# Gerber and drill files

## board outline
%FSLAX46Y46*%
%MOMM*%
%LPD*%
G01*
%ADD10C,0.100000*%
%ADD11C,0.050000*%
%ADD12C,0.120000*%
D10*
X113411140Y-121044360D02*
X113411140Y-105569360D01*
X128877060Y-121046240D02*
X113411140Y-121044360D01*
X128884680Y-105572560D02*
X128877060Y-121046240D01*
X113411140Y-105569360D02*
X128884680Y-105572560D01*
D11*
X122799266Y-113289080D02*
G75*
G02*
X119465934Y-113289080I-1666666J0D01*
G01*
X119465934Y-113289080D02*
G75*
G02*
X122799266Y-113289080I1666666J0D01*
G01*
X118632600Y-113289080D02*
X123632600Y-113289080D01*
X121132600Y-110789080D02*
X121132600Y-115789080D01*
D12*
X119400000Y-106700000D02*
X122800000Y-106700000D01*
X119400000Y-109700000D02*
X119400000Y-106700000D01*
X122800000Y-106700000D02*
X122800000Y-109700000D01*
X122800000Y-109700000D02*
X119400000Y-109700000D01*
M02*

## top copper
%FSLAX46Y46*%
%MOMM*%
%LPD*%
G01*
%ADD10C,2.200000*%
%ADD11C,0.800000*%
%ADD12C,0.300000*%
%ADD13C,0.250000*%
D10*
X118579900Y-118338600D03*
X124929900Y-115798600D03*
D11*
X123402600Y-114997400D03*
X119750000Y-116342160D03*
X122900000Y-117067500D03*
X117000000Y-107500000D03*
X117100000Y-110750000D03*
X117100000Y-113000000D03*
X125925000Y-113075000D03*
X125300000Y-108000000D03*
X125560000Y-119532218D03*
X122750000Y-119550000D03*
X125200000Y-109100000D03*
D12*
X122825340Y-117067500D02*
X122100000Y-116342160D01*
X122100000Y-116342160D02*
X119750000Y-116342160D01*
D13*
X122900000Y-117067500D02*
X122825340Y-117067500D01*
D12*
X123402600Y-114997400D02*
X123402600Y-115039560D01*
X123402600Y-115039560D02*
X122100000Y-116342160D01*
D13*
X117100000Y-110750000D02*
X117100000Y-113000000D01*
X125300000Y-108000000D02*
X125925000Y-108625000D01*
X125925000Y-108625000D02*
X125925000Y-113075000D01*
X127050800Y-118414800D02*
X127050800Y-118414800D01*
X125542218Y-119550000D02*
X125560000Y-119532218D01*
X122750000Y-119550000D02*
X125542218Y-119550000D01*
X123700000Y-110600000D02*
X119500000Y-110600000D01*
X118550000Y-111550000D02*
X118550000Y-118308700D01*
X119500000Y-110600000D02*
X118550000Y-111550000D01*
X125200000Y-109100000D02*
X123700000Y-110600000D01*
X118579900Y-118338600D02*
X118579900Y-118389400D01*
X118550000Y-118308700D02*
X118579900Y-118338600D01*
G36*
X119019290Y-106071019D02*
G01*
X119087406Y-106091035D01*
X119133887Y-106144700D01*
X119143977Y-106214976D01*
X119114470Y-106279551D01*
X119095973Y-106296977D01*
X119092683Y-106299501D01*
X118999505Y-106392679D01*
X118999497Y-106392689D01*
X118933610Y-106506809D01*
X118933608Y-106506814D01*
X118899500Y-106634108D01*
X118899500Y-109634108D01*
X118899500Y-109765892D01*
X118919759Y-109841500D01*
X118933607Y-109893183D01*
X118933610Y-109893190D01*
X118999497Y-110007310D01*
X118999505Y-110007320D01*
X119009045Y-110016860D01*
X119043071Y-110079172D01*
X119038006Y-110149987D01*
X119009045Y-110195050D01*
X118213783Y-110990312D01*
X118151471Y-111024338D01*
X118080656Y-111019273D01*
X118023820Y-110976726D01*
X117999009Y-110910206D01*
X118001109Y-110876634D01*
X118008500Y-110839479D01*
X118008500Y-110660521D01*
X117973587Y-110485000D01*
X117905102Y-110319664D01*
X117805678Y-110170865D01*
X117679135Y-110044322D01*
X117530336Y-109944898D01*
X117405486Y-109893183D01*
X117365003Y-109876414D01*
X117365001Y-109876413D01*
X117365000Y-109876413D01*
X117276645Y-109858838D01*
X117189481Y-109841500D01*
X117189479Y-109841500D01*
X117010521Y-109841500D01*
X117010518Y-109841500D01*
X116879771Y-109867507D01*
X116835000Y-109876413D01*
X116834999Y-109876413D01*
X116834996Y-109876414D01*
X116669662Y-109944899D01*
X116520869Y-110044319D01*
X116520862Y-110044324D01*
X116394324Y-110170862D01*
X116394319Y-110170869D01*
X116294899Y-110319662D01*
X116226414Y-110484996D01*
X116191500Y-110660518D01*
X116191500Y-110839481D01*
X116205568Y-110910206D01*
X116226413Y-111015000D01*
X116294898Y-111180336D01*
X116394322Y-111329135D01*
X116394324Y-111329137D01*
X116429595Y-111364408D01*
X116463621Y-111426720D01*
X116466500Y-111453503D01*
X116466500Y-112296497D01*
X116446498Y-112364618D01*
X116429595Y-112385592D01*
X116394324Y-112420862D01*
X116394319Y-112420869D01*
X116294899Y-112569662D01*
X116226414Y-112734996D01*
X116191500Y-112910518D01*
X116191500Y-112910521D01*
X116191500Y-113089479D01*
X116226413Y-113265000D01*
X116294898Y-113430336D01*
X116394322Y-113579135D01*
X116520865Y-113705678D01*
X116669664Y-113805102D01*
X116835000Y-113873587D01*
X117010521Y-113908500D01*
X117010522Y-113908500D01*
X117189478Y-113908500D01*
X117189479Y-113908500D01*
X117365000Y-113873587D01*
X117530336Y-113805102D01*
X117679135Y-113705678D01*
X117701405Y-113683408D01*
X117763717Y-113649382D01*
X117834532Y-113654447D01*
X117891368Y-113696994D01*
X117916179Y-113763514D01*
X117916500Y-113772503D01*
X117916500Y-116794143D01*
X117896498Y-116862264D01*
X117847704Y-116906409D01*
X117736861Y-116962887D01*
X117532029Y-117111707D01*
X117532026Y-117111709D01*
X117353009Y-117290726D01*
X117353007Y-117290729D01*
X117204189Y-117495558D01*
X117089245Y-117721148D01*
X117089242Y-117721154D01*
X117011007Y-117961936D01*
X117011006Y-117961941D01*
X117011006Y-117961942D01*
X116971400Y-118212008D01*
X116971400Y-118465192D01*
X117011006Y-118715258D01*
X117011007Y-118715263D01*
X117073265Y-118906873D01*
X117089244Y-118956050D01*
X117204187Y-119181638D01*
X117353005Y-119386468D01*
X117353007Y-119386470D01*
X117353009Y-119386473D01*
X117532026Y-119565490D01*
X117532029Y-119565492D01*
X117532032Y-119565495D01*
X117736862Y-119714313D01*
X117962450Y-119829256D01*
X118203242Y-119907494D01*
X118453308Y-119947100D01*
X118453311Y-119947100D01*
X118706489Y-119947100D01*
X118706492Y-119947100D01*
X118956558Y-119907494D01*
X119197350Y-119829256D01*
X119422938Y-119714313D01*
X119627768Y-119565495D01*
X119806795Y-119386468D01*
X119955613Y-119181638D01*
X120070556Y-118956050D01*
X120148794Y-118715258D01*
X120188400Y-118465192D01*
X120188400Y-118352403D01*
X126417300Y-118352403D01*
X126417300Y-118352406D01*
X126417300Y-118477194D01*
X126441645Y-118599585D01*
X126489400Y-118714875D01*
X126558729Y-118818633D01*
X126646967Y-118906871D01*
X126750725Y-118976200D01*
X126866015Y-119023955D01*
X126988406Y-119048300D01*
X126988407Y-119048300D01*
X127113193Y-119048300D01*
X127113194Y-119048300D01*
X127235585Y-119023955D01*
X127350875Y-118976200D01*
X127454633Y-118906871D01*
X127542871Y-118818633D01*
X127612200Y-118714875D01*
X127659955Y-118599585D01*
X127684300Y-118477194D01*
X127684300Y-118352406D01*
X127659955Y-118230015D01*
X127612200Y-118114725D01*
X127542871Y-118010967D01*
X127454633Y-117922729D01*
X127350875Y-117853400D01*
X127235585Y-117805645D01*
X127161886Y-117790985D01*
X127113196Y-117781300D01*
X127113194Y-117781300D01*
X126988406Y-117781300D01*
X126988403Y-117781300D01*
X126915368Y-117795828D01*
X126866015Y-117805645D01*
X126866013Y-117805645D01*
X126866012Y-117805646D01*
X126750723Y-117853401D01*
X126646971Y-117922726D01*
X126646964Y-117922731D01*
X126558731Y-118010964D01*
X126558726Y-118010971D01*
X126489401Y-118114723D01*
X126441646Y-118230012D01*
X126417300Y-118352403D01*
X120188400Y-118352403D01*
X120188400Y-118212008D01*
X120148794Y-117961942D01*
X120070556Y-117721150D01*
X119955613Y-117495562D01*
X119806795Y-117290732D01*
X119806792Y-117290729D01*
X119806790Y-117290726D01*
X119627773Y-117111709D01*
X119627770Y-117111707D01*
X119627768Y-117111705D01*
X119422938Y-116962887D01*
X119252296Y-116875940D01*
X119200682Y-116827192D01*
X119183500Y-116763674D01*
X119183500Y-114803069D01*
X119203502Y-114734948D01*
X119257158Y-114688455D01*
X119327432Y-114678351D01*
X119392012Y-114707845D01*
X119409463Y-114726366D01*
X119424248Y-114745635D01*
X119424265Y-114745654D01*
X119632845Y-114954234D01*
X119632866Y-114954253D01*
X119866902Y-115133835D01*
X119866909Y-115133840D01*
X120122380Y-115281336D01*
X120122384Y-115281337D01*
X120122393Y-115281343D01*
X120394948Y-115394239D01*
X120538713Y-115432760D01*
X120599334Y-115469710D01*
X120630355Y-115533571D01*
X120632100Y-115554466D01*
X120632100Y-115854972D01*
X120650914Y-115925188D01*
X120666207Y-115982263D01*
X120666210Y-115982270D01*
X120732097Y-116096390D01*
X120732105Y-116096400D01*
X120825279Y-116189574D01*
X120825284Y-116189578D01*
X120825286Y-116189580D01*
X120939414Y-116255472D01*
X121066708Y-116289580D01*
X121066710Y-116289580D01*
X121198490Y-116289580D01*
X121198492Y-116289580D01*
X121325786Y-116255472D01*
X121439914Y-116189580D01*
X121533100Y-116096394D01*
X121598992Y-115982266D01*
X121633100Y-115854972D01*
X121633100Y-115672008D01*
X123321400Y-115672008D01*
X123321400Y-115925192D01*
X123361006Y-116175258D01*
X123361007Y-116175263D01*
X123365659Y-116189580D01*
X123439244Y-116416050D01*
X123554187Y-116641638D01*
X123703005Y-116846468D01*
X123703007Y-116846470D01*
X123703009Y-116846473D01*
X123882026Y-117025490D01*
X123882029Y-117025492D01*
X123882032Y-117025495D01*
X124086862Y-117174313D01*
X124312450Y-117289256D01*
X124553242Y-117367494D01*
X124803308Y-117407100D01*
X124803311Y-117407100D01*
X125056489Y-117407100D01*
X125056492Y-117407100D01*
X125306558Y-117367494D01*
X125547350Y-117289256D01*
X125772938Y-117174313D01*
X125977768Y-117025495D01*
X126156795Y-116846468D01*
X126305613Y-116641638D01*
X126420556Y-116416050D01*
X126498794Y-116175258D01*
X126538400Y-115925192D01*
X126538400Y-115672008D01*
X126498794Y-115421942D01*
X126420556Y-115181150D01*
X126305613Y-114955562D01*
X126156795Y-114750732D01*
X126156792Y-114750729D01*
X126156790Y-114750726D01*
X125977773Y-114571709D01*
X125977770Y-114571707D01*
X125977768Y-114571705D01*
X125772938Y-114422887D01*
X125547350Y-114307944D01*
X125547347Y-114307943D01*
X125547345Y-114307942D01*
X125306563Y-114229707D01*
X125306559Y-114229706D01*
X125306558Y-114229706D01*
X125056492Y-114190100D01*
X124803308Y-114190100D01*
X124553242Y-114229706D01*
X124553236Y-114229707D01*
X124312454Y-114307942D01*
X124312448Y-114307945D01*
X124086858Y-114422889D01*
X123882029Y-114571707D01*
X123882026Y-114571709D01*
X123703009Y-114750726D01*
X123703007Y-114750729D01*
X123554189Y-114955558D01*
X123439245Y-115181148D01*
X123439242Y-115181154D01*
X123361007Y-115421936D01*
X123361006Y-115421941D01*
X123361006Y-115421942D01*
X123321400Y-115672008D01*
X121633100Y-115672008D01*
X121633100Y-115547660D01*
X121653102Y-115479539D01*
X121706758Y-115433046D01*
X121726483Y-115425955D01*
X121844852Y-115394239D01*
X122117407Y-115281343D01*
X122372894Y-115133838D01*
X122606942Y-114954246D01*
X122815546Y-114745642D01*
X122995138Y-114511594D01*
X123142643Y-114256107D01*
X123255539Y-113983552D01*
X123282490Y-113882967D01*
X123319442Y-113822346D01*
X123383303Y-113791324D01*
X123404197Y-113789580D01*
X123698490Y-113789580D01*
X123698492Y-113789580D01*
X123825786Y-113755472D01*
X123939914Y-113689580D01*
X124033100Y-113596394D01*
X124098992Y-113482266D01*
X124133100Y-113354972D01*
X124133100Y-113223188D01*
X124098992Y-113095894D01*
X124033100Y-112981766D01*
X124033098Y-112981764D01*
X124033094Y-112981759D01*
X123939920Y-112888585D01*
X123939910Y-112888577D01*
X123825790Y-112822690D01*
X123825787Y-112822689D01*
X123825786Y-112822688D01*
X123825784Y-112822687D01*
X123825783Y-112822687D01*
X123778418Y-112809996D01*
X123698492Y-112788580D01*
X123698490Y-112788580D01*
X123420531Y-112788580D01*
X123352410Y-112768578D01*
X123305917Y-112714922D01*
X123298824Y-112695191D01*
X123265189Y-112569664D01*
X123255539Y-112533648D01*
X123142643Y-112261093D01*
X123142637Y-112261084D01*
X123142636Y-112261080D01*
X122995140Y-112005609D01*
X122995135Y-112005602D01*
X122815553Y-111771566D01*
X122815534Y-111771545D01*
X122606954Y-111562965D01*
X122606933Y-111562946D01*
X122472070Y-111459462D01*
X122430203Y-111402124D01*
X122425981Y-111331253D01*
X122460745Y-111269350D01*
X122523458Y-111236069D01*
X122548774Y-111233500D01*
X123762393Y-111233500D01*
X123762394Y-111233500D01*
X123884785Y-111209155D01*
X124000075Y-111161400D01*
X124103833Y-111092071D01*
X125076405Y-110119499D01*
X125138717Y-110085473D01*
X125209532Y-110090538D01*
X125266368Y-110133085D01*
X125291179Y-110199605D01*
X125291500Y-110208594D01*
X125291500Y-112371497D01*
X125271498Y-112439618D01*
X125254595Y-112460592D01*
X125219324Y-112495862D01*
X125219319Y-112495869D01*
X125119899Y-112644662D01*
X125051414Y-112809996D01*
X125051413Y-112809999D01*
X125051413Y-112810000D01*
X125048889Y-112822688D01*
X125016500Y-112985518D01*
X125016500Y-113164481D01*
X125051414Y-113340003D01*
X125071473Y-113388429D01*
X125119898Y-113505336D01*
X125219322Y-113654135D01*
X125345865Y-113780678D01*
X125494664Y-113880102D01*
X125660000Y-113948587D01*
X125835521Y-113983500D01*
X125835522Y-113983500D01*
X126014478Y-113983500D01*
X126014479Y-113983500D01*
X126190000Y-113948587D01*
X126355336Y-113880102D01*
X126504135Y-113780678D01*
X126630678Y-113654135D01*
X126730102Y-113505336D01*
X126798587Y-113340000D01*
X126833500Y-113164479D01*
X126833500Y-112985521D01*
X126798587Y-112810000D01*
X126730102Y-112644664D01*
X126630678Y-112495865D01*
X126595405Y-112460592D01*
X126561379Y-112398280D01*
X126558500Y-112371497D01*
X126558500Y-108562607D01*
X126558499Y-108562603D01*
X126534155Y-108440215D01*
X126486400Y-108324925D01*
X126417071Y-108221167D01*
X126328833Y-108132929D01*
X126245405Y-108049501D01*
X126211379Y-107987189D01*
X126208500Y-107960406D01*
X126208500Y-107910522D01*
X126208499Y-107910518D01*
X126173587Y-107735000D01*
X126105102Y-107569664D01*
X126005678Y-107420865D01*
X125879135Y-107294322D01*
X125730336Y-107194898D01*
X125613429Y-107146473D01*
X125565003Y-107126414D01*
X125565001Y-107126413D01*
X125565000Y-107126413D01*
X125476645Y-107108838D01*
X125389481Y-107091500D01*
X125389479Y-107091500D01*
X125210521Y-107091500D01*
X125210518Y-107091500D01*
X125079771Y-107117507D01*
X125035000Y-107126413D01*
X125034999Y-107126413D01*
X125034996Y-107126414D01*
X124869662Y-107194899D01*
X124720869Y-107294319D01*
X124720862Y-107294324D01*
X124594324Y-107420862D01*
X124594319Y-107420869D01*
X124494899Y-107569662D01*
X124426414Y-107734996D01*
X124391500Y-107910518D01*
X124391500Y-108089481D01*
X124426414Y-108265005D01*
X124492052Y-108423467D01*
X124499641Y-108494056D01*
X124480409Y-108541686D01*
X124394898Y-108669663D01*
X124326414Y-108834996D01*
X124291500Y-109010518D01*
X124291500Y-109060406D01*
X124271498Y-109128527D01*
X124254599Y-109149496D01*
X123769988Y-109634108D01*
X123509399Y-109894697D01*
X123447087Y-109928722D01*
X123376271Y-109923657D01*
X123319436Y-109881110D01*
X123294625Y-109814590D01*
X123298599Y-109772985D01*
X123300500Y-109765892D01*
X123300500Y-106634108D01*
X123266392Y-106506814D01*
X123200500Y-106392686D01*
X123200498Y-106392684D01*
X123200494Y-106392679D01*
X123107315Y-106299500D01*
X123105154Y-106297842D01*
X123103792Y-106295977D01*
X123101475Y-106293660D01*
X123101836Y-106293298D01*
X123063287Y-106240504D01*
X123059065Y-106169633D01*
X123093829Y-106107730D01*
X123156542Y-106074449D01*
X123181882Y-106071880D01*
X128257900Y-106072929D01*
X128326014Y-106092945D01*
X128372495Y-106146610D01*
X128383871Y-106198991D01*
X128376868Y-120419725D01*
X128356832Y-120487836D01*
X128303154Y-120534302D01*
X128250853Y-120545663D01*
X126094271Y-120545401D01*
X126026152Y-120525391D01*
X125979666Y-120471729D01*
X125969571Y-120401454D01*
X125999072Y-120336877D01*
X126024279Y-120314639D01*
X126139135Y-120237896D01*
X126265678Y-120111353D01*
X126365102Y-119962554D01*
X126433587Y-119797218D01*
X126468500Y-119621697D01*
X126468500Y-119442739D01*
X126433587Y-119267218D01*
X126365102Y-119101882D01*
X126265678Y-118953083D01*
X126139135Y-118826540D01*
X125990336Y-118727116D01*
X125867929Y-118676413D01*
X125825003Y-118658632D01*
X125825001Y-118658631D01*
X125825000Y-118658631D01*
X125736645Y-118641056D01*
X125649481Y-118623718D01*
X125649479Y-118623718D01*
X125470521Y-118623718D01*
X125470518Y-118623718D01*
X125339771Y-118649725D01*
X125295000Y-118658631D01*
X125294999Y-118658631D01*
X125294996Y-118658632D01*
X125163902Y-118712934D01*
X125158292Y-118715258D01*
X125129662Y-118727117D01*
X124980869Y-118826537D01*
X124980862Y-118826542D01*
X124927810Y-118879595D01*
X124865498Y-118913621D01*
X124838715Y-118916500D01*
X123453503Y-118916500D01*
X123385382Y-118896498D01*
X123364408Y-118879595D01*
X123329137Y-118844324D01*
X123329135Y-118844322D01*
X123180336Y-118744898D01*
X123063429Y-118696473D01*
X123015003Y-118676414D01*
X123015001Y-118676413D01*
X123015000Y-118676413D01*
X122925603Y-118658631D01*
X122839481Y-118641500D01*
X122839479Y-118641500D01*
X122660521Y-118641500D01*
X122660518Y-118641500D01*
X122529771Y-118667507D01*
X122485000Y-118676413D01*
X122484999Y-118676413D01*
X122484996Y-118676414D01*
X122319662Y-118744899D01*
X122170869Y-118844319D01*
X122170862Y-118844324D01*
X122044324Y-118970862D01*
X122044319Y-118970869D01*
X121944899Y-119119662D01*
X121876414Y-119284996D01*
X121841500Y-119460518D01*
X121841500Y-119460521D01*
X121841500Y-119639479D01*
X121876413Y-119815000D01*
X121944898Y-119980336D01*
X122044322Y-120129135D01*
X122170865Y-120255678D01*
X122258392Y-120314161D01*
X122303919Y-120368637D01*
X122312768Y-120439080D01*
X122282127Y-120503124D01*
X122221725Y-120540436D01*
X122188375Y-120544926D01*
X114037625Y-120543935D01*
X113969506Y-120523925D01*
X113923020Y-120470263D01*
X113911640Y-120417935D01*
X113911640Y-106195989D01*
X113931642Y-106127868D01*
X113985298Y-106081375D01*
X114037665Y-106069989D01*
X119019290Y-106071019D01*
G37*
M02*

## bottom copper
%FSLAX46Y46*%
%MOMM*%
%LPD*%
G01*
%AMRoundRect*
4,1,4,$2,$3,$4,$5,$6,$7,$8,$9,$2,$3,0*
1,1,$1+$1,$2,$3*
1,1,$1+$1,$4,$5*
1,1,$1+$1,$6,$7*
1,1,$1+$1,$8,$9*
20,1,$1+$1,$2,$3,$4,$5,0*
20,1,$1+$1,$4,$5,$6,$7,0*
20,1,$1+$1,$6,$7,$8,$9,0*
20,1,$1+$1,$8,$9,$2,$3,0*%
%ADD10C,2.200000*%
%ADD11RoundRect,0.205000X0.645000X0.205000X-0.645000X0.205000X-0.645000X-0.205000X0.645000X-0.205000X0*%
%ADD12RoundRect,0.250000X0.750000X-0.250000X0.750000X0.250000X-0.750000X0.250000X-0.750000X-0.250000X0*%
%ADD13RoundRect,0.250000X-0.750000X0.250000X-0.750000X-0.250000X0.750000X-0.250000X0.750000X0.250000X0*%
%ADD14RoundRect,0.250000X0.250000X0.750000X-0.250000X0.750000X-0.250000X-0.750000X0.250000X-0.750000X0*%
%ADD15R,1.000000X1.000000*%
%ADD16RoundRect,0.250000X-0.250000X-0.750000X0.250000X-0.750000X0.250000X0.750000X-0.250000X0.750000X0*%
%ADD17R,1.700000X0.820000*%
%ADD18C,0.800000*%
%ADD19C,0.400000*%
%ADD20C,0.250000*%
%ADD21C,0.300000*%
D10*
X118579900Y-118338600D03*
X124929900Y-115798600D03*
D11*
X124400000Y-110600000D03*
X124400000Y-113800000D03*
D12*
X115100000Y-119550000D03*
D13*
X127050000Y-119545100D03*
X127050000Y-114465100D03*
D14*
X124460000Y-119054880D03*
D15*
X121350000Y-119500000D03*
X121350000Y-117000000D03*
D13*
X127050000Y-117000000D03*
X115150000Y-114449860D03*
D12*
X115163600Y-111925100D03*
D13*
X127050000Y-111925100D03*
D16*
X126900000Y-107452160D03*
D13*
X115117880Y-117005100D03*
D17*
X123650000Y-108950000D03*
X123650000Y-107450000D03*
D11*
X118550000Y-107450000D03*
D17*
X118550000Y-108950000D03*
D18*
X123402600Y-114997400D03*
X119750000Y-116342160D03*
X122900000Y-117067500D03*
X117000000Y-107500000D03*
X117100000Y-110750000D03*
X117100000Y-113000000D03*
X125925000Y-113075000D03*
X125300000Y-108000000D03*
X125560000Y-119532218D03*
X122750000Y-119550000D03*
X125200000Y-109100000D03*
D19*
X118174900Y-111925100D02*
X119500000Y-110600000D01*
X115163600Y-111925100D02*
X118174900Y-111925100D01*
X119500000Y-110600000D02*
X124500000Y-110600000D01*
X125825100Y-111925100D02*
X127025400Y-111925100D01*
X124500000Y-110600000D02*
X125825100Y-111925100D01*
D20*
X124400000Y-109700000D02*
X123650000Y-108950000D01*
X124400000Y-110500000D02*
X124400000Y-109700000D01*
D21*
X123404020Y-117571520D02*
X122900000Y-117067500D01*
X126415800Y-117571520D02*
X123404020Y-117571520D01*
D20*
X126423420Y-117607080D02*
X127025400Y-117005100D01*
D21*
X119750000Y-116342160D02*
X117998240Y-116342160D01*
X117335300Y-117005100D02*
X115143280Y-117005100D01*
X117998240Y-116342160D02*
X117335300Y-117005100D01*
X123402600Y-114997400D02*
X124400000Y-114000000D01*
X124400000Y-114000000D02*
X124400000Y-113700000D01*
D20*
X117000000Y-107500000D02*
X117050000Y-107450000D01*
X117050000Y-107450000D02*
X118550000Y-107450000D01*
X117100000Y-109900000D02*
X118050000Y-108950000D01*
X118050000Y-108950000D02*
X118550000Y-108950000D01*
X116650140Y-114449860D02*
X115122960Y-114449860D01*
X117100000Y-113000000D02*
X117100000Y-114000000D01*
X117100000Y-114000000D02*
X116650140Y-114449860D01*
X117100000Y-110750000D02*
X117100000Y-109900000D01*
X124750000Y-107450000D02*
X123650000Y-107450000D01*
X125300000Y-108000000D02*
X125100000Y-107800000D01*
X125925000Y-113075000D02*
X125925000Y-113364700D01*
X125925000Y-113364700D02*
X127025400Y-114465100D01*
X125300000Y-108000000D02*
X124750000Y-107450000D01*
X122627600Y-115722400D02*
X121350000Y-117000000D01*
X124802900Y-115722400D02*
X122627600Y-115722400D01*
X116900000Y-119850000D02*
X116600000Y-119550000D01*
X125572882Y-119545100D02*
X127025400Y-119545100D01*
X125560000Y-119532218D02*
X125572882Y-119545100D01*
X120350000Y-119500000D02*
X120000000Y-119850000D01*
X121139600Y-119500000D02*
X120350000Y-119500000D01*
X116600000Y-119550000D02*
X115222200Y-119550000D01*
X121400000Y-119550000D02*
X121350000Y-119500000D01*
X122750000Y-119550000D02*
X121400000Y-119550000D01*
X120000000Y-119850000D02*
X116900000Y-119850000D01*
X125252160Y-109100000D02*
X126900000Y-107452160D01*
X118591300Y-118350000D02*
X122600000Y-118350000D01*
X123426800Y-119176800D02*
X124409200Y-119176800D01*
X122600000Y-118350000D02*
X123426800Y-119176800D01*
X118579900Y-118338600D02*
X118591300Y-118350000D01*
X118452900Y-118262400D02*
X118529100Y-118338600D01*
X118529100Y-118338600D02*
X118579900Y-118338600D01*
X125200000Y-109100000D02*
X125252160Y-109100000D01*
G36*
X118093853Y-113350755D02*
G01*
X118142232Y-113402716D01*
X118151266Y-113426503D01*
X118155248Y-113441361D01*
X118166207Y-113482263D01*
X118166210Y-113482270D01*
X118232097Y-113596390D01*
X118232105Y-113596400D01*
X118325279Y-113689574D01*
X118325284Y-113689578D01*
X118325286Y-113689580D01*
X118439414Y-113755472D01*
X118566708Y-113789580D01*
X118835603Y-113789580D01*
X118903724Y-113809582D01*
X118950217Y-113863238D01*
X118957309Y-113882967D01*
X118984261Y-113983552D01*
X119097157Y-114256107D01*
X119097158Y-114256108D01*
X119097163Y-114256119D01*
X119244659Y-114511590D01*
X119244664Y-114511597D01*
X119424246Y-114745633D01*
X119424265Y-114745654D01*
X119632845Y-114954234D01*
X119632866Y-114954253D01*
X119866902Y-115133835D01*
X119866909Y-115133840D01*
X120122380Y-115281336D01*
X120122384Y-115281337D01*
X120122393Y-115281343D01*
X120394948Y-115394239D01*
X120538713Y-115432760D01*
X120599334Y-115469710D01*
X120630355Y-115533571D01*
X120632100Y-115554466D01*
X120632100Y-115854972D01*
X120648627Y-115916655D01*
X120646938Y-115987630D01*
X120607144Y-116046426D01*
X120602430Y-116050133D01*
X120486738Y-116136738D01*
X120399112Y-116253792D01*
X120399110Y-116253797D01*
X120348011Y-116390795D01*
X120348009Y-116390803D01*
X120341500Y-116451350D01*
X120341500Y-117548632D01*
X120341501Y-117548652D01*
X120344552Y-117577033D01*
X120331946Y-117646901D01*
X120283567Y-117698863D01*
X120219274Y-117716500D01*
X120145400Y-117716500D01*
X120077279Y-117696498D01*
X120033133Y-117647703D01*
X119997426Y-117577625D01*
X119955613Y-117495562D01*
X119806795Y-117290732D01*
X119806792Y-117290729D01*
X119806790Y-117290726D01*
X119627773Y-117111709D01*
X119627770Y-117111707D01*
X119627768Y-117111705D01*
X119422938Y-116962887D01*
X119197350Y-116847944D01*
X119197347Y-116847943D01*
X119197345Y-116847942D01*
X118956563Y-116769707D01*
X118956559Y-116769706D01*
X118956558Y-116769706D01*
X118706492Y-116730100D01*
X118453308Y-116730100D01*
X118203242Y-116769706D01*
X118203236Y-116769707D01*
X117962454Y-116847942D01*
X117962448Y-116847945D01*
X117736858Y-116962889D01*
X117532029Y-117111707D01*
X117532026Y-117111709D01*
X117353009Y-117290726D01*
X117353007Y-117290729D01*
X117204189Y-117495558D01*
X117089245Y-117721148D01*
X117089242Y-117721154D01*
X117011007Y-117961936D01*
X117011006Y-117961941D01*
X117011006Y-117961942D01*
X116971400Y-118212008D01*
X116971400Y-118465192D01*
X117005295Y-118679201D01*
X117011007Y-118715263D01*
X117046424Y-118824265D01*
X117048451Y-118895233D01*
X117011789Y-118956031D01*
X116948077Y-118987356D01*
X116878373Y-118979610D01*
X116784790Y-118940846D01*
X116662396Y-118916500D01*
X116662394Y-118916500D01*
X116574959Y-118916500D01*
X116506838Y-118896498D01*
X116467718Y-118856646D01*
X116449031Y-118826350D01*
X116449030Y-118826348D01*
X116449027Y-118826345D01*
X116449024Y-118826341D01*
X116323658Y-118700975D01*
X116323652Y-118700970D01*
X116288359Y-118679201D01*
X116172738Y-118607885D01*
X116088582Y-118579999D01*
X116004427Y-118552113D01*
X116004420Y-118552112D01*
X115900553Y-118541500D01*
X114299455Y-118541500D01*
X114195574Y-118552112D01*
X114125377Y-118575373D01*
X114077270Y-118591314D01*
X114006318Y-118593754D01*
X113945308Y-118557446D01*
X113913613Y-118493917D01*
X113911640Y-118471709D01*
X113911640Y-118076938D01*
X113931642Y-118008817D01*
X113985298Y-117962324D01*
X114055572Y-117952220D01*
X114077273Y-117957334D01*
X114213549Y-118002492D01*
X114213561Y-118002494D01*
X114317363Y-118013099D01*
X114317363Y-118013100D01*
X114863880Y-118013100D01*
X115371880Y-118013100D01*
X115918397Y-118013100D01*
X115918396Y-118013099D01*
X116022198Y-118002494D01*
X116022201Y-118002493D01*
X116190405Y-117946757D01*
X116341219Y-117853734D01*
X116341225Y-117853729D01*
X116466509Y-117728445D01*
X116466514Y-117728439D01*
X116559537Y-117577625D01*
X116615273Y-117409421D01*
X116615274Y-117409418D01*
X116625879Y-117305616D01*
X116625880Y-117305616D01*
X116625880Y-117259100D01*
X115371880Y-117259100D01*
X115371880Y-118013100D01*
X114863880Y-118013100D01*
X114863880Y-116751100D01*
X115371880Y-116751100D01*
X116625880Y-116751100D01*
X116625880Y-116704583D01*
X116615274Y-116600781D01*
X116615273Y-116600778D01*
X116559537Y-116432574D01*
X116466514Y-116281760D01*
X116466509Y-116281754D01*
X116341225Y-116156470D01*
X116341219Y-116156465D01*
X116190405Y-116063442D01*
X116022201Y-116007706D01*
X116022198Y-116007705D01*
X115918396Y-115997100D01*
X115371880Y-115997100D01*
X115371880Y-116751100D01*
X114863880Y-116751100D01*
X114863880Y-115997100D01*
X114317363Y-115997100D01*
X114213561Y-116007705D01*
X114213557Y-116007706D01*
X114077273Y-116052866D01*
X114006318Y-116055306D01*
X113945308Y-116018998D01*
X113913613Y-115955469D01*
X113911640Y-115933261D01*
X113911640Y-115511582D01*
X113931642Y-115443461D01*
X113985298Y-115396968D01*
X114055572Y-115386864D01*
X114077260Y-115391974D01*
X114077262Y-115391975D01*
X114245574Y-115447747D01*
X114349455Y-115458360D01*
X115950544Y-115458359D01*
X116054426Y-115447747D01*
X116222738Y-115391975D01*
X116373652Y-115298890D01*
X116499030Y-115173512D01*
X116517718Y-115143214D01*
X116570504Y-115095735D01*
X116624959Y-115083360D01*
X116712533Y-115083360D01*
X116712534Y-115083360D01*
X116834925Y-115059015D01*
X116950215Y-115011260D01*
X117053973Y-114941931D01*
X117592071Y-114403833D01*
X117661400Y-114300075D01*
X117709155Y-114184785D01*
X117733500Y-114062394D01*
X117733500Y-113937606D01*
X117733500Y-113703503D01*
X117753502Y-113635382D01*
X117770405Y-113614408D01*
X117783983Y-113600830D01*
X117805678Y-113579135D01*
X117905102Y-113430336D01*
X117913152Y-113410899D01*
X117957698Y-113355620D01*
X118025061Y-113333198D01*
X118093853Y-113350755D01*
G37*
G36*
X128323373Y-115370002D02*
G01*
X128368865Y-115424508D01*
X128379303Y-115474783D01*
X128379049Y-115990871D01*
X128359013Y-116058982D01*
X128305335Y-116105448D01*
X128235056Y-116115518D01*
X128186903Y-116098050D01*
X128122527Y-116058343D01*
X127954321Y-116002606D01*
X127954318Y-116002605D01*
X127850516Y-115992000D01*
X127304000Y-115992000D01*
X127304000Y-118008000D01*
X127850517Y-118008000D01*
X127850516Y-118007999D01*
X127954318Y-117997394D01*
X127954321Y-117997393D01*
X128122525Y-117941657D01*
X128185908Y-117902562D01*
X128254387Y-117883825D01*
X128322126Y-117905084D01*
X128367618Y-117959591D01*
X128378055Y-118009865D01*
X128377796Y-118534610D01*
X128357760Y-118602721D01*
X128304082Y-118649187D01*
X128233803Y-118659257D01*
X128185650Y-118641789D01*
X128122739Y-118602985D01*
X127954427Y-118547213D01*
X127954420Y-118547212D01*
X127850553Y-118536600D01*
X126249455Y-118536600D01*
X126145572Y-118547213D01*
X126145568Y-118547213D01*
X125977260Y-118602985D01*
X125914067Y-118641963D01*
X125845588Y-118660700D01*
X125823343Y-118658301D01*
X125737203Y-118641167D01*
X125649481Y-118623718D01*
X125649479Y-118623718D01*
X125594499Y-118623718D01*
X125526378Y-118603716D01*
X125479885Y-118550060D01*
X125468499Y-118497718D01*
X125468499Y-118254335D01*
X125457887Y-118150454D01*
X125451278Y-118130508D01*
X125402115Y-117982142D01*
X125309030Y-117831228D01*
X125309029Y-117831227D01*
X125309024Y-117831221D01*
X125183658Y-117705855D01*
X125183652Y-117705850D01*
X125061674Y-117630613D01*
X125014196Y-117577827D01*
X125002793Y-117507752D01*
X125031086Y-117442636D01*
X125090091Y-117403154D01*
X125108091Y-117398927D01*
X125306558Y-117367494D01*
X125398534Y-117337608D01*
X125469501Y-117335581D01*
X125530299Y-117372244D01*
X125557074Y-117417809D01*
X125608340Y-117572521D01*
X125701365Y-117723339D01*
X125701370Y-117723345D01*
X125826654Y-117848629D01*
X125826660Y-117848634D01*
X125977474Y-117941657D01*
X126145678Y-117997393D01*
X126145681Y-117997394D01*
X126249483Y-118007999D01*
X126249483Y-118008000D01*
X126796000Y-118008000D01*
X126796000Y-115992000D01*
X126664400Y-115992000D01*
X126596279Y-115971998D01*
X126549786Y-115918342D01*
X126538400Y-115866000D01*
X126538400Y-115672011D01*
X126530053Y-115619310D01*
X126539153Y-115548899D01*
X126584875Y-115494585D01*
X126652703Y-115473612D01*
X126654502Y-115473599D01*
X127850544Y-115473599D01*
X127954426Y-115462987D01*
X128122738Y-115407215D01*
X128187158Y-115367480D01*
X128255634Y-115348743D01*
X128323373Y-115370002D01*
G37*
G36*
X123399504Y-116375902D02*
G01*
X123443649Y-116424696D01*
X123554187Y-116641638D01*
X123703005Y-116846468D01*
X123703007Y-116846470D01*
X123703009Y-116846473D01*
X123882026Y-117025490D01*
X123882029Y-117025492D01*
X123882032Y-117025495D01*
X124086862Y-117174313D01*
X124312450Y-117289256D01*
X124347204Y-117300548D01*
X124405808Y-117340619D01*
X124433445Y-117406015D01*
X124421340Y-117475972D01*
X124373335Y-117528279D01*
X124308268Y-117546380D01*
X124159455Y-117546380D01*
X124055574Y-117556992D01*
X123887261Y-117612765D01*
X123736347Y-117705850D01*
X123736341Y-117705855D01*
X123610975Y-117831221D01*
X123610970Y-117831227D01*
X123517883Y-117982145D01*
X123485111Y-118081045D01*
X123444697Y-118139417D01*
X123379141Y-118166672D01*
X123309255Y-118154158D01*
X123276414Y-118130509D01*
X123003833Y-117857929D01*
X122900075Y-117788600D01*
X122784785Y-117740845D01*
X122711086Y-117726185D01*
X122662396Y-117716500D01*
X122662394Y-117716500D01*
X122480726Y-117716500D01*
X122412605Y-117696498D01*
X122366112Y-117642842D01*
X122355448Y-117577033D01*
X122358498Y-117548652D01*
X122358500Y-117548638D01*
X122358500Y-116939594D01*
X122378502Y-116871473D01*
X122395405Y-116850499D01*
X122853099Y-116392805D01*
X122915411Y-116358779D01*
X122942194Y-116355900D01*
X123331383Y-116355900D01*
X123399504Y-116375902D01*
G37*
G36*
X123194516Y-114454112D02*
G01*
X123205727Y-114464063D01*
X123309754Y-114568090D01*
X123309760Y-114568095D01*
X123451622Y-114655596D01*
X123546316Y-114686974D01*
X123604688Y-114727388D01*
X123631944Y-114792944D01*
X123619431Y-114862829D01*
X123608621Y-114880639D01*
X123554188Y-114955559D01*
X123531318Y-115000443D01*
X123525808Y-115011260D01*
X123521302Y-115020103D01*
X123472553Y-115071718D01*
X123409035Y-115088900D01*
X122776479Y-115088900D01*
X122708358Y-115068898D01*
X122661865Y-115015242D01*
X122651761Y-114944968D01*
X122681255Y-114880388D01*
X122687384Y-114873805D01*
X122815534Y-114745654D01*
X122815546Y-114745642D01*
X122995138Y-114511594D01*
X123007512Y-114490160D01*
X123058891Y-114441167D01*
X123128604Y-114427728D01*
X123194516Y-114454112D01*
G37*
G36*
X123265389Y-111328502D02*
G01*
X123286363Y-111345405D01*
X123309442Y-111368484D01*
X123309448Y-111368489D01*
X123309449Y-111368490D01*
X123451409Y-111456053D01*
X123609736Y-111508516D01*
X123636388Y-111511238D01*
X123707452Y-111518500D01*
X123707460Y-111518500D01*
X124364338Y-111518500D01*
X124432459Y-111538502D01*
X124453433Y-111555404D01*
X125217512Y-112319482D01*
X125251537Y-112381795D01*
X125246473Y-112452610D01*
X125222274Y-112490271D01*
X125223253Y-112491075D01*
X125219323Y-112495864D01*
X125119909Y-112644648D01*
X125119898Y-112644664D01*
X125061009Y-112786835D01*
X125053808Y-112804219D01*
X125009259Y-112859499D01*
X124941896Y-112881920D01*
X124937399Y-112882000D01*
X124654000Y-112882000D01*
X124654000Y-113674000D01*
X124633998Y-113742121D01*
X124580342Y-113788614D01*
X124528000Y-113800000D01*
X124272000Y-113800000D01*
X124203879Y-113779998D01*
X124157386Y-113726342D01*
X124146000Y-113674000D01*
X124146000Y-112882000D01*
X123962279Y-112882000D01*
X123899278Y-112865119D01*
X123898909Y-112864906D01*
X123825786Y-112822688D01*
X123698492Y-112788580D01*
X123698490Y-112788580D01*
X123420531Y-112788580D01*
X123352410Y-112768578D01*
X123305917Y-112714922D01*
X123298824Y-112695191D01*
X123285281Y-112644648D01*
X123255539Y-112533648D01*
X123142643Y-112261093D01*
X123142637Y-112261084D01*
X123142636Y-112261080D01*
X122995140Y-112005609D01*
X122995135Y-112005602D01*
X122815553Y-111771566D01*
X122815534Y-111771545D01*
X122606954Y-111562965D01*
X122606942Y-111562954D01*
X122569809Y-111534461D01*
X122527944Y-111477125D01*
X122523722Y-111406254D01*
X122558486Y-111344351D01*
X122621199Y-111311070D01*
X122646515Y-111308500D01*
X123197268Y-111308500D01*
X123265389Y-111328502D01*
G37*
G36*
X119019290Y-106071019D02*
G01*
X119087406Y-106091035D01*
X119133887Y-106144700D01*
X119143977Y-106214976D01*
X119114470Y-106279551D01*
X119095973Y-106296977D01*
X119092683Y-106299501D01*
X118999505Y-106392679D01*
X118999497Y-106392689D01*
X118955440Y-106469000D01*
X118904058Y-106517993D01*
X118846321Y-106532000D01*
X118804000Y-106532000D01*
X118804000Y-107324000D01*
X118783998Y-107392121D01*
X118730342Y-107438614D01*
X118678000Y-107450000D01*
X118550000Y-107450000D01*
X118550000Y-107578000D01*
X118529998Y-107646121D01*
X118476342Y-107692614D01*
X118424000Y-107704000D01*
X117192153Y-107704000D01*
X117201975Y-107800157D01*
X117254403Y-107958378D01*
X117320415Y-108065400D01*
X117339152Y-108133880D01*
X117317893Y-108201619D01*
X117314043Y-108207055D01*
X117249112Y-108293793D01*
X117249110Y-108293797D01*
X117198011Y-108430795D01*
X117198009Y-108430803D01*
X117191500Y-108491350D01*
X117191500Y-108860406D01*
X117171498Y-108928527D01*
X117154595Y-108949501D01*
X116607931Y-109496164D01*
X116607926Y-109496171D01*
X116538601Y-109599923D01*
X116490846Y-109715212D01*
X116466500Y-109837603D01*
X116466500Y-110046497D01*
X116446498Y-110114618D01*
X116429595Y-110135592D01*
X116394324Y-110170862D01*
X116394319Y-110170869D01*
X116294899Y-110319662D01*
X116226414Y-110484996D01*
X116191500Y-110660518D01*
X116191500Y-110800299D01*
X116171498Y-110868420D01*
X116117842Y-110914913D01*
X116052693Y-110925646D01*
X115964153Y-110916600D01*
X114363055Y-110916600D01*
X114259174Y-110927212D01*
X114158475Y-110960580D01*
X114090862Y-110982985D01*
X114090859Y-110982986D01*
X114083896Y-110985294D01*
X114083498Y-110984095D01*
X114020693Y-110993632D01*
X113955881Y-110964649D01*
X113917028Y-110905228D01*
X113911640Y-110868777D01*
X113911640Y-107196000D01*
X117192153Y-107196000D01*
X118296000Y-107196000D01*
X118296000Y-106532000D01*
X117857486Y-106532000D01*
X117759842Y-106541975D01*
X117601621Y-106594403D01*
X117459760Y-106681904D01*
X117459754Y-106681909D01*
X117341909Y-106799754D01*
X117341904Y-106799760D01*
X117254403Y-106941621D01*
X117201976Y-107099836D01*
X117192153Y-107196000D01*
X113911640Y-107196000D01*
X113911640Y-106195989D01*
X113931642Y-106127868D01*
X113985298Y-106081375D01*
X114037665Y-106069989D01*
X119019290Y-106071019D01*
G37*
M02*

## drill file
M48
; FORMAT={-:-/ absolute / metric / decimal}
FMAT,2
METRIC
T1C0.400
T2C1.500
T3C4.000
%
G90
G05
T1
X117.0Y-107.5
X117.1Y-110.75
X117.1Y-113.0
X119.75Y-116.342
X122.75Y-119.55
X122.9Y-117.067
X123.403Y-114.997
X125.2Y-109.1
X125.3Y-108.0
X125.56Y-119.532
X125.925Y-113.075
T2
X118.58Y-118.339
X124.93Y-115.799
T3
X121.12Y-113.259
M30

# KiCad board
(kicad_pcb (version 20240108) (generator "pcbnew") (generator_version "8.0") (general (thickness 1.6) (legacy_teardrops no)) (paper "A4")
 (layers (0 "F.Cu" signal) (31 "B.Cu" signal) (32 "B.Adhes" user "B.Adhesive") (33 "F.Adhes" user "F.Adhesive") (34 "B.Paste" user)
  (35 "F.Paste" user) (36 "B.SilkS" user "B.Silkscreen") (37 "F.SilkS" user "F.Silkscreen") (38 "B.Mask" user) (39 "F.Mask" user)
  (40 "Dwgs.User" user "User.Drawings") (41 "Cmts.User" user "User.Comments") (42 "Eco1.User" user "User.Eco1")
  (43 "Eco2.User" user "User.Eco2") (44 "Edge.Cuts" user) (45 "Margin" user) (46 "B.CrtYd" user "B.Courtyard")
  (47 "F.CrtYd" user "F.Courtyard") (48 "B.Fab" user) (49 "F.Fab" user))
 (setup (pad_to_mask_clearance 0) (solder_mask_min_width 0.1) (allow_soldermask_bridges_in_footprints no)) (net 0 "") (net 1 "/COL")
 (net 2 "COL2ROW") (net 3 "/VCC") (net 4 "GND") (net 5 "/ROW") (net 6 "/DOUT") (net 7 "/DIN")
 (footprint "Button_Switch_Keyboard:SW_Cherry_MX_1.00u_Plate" (layer "F.Cu") (at 118.5799 118.3386 180)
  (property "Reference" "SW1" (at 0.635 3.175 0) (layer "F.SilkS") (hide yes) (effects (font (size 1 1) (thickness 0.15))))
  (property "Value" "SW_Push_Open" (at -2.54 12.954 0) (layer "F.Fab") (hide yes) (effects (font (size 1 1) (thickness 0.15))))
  (pad "" np_thru_hole circle (at -2.54 5.08 180) (size 4 4) (drill 4) (layers "*.Cu" "*.Mask"))
  (pad "1" thru_hole circle (at 0 0 180) (size 2.2 2.2) (drill 1.5) (layers "*.Cu" "*.Mask") (remove_unused_layers no) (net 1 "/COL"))
  (pad "2" thru_hole circle (at -6.35 2.54 180) (size 2.2 2.2) (drill 1.5) (layers "*.Cu" "*.Mask") (remove_unused_layers no)
   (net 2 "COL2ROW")))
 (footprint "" (layer "F.Cu") (at 124.4 110.6)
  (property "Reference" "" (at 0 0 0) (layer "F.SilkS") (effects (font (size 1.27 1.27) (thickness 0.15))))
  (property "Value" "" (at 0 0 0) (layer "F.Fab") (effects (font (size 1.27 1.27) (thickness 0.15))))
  (pad "3" smd roundrect (at 0 0 180) (size 1.7 0.82) (layers "B.Cu" "B.Paste" "B.Mask") (roundrect_rratio 0.25) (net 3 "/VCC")))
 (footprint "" (layer "F.Cu") (at 124.4 113.8)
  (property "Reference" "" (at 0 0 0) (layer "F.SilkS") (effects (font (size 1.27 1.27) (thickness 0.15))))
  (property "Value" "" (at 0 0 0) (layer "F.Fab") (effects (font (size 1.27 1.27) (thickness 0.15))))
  (pad "3" smd roundrect (at 0 0 180) (size 1.7 0.82) (layers "B.Cu" "B.Paste" "B.Mask") (roundrect_rratio 0.25) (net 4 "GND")))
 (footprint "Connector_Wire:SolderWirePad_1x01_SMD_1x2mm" (layer "B.Cu") (at 115.1 119.55 90)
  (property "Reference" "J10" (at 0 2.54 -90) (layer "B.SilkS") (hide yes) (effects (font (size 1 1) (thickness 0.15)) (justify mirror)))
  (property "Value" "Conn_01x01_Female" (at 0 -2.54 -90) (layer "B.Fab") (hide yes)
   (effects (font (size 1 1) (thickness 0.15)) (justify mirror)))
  (pad "1" smd roundrect (at 0 0 90) (size 1 2) (layers "B.Cu" "B.Paste" "B.Mask") (roundrect_rratio 0.25) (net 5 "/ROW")))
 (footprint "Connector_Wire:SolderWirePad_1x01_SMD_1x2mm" (layer "B.Cu") (at 127.05 119.5451 -90)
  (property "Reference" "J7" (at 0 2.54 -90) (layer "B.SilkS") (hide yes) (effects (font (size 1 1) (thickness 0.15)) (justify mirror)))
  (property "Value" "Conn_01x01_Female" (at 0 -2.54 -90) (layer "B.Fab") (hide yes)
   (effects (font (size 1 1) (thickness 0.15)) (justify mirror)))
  (pad "1" smd roundrect (at 0 0 270) (size 1 2) (layers "B.Cu" "B.Paste" "B.Mask") (roundrect_rratio 0.25) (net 5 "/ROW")))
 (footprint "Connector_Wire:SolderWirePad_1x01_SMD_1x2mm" (layer "B.Cu") (at 127.05 114.4651 -90)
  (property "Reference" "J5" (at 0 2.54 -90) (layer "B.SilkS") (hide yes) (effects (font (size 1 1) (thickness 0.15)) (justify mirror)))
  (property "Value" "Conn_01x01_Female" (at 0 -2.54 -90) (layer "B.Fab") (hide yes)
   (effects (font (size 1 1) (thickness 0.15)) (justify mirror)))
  (pad "1" smd roundrect (at 0 0 270) (size 1 2) (layers "B.Cu" "B.Paste" "B.Mask") (roundrect_rratio 0.25) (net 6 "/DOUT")))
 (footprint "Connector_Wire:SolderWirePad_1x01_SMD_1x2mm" (layer "B.Cu") (at 124.46 119.05488 180)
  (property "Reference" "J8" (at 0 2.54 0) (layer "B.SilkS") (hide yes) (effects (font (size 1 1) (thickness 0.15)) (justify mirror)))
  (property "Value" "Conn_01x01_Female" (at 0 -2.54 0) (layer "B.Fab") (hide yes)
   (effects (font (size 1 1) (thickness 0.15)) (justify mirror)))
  (pad "1" smd roundrect (at 0 0 180) (size 1 2) (layers "B.Cu" "B.Paste" "B.Mask") (roundrect_rratio 0.25) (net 1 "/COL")))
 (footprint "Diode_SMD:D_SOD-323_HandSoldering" (layer "B.Cu") (at 121.35 118.25 90)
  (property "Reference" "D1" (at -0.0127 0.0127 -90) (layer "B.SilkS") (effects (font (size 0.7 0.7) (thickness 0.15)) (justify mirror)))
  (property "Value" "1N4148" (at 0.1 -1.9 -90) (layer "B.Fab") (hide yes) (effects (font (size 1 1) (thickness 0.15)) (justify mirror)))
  (pad "1" smd rect (at -1.25 0 90) (size 1 1) (layers "B.Cu" "B.Paste" "B.Mask") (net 5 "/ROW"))
  (pad "2" smd rect (at 1.25 0 90) (size 1 1) (layers "B.Cu" "B.Paste" "B.Mask") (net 2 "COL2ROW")))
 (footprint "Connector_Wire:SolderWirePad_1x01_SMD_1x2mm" (layer "B.Cu") (at 127.05 117 -90)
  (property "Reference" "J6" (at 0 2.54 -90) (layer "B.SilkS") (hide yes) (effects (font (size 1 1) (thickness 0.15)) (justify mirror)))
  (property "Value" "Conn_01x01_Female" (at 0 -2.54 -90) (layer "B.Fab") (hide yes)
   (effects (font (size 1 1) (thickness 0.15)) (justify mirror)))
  (pad "1" smd roundrect (at 0 0 270) (size 1 2) (layers "B.Cu" "B.Paste" "B.Mask") (roundrect_rratio 0.25) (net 4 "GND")))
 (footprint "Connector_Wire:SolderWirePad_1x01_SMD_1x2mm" (layer "B.Cu") (at 115.15 114.44986 -90)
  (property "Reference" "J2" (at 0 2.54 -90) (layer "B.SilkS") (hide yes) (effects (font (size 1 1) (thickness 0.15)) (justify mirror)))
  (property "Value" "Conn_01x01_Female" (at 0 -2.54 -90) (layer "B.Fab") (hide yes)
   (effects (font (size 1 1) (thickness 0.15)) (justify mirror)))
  (pad "1" smd roundrect (at 0 0 270) (size 1 2) (layers "B.Cu" "B.Paste" "B.Mask") (roundrect_rratio 0.25) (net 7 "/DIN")))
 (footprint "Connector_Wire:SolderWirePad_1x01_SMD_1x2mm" (layer "B.Cu") (at 115.1636 111.9251 90)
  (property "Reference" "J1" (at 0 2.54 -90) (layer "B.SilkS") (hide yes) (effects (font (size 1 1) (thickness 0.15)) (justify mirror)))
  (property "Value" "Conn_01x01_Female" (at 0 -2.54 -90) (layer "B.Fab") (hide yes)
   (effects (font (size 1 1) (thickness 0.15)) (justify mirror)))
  (pad "1" smd roundrect (at 0 0 90) (size 1 2) (layers "B.Cu" "B.Paste" "B.Mask") (roundrect_rratio 0.25) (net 3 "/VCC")))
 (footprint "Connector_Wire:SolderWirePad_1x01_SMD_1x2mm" (layer "B.Cu") (at 127.05 111.9251 -90)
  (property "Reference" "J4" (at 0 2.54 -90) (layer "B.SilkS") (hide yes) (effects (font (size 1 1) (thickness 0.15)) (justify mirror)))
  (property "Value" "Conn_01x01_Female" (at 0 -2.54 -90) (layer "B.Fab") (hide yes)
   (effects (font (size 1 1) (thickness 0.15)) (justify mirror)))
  (pad "1" smd roundrect (at 0 0 270) (size 1 2) (layers "B.Cu" "B.Paste" "B.Mask") (roundrect_rratio 0.25) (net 3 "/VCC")))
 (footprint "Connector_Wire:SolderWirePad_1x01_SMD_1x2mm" (layer "B.Cu") (at 126.9 107.45216)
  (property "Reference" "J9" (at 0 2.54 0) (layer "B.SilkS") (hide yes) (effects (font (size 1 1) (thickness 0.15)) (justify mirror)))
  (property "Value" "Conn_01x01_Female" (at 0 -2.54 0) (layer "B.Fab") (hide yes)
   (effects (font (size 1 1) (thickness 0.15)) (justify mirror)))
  (pad "1" smd roundrect (at 0 0) (size 1 2) (layers "B.Cu" "B.Paste" "B.Mask") (roundrect_rratio 0.25) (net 1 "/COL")))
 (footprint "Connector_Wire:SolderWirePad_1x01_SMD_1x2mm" (layer "B.Cu") (at 115.11788 117.0051 -90)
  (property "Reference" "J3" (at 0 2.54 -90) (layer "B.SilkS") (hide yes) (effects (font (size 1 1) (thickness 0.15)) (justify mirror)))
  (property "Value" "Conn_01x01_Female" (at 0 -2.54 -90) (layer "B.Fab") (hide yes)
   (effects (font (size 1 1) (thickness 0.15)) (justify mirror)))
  (pad "1" smd roundrect (at 0 0 270) (size 1 2) (layers "B.Cu" "B.Paste" "B.Mask") (roundrect_rratio 0.25) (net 4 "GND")))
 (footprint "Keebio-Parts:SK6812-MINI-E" (layer "B.Cu") (at 121.1 108.2 180)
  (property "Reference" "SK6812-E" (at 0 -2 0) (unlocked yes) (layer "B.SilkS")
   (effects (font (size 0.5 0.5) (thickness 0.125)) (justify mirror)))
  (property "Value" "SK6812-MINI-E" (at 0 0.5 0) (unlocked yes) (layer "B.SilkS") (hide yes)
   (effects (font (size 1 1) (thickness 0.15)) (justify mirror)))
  (fp_line (start 1.7 1.5) (end -1.7 1.5) (stroke (width 0.12) (type solid)) (layer "Edge.Cuts"))
  (fp_line (start 1.7 -1.5) (end 1.7 1.5) (stroke (width 0.12) (type solid)) (layer "Edge.Cuts"))
  (fp_line (start -1.7 1.5) (end -1.7 -1.5) (stroke (width 0.12) (type solid)) (layer "Edge.Cuts"))
  (fp_line (start -1.7 -1.5) (end 1.7 -1.5) (stroke (width 0.12) (type solid)) (layer "Edge.Cuts"))
  (pad "1" smd rect (at -2.55 -0.75 180) (size 1.7 0.82) (layers "B.Cu" "B.Paste" "B.Mask") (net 3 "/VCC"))
  (pad "2" smd rect (at -2.55 0.75 180) (size 1.7 0.82) (layers "B.Cu" "B.Paste" "B.Mask") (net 6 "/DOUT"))
  (pad "3" smd roundrect (at 2.55 0.75 180) (size 1.7 0.82) (layers "B.Cu" "B.Paste" "B.Mask") (roundrect_rratio 0.25) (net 4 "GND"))
  (pad "4" smd rect (at 2.55 -0.75 180) (size 1.7 0.82) (layers "B.Cu" "B.Paste" "B.Mask") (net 7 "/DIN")))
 (gr_line (start 113.41114 121.04436) (end 113.41114 105.56936) (stroke (width 0.1) (type solid)) (layer "Edge.Cuts"))
 (gr_line (start 128.87706 121.04624) (end 113.41114 121.04436) (stroke (width 0.1) (type solid)) (layer "Edge.Cuts"))
 (gr_line (start 128.88468 105.57256) (end 128.87706 121.04624) (stroke (width 0.1) (type solid)) (layer "Edge.Cuts"))
 (gr_line (start 113.41114 105.56936) (end 128.88468 105.57256) (stroke (width 0.1) (type solid)) (layer "Edge.Cuts"))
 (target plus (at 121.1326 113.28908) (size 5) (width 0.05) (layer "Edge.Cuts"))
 (segment (start 118.1749 111.9251) (end 119.5 110.6) (width 0.4) (layer "B.Cu") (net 3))
 (segment (start 115.1636 111.9251) (end 118.1749 111.9251) (width 0.4) (layer "B.Cu") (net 3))
 (segment (start 119.5 110.6) (end 124.5 110.6) (width 0.4) (layer "B.Cu") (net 3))
 (segment (start 125.8251 111.9251) (end 127.0254 111.9251) (width 0.4) (layer "B.Cu") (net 3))
 (segment (start 124.5 110.6) (end 125.8251 111.9251) (width 0.4) (layer "B.Cu") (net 3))
 (segment (start 124.4 109.7) (end 123.65 108.95) (width 0.25) (layer "B.Cu") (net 3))
 (segment (start 124.4 110.5) (end 124.4 109.7) (width 0.25) (layer "B.Cu") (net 3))
 (segment (start 122.82534 117.0675) (end 122.1 116.34216) (width 0.3) (layer "F.Cu") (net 4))
 (segment (start 122.1 116.34216) (end 119.75 116.34216) (width 0.3) (layer "F.Cu") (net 4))
 (segment (start 122.9 117.0675) (end 122.82534 117.0675) (width 0.25) (layer "F.Cu") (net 4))
 (segment (start 123.4026 114.9974) (end 123.4026 115.03956) (width 0.3) (layer "F.Cu") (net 4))
 (segment (start 123.4026 115.03956) (end 122.1 116.34216) (width 0.3) (layer "F.Cu") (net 4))
 (via (at 123.4026 114.9974) (size 0.8) (drill 0.4) (layers "F.Cu" "B.Cu") (free yes) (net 4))
 (via (at 119.75 116.34216) (size 0.8) (drill 0.4) (layers "F.Cu" "B.Cu") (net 4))
 (via (at 122.9 117.0675) (size 0.8) (drill 0.4) (layers "F.Cu" "B.Cu") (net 4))
 (via (at 117 107.5) (size 0.8) (drill 0.4) (layers "F.Cu" "B.Cu") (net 4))
 (segment (start 123.40402 117.57152) (end 122.9 117.0675) (width 0.3) (layer "B.Cu") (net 4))
 (segment (start 126.4158 117.57152) (end 123.40402 117.57152) (width 0.3) (layer "B.Cu") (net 4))
 (segment (start 126.42342 117.60708) (end 127.0254 117.0051) (width 0.25) (layer "B.Cu") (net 4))
 (segment (start 119.75 116.34216) (end 117.99824 116.34216) (width 0.3) (layer "B.Cu") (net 4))
 (segment (start 117.3353 117.0051) (end 115.14328 117.0051) (width 0.3) (layer "B.Cu") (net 4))
 (segment (start 117.99824 116.34216) (end 117.3353 117.0051) (width 0.3) (layer "B.Cu") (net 4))
 (segment (start 123.4026 114.9974) (end 124.4 114) (width 0.3) (layer "B.Cu") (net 4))
 (segment (start 124.4 114) (end 124.4 113.7) (width 0.3) (layer "B.Cu") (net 4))
 (segment (start 117 107.5) (end 117.05 107.45) (width 0.25) (layer "B.Cu") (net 4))
 (segment (start 117.05 107.45) (end 118.55 107.45) (width 0.25) (layer "B.Cu") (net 4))
 (segment (start 117.1 110.75) (end 117.1 113) (width 0.25) (layer "F.Cu") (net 7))
 (via (at 117.1 110.75) (size 0.8) (drill 0.4) (layers "F.Cu" "B.Cu") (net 7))
 (via (at 117.1 113) (size 0.8) (drill 0.4) (layers "F.Cu" "B.Cu") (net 7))
 (segment (start 117.1 109.9) (end 118.05 108.95) (width 0.25) (layer "B.Cu") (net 7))
 (segment (start 118.05 108.95) (end 118.55 108.95) (width 0.25) (layer "B.Cu") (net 7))
 (segment (start 116.65014 114.44986) (end 115.12296 114.44986) (width 0.25) (layer "B.Cu") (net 7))
 (segment (start 117.1 113) (end 117.1 114) (width 0.25) (layer "B.Cu") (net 7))
 (segment (start 117.1 114) (end 116.65014 114.44986) (width 0.25) (layer "B.Cu") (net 7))
 (segment (start 117.1 110.75) (end 117.1 109.9) (width 0.25) (layer "B.Cu") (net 7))
 (segment (start 125.3 108) (end 125.925 108.625) (width 0.25) (layer "F.Cu") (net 6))
 (segment (start 125.925 108.625) (end 125.925 113.075) (width 0.25) (layer "F.Cu") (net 6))
 (via (at 125.925 113.075) (size 0.8) (drill 0.4) (layers "F.Cu" "B.Cu") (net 6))
 (via (at 125.3 108) (size 0.8) (drill 0.4) (layers "F.Cu" "B.Cu") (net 6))
 (segment (start 124.75 107.45) (end 123.65 107.45) (width 0.25) (layer "B.Cu") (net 6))
 (segment (start 125.3 108) (end 125.1 107.8) (width 0.25) (layer "B.Cu") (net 6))
 (segment (start 125.925 113.075) (end 125.925 113.3647) (width 0.25) (layer "B.Cu") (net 6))
 (segment (start 125.925 113.3647) (end 127.0254 114.4651) (width 0.25) (layer "B.Cu") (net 6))
 (segment (start 125.3 108) (end 124.75 107.45) (width 0.25) (layer "B.Cu") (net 6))
 (segment (start 122.6276 115.7224) (end 121.35 117) (width 0.25) (layer "B.Cu") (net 2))
 (segment (start 124.8029 115.7224) (end 122.6276 115.7224) (width 0.25) (layer "B.Cu") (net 2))
 (segment (start 127.0508 118.4148) (end 127.0508 118.4148) (width 0.25) (layer "F.Cu") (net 5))
 (segment (start 125.542218 119.55) (end 125.56 119.532218) (width 0.25) (layer "F.Cu") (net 5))
 (segment (start 122.75 119.55) (end 125.542218 119.55) (width 0.25) (layer "F.Cu") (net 5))
 (via (at 125.56 119.532218) (size 0.8) (drill 0.4) (layers "F.Cu" "B.Cu") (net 5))
 (via (at 122.75 119.55) (size 0.8) (drill 0.4) (layers "F.Cu" "B.Cu") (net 5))
 (segment (start 116.9 119.85) (end 116.6 119.55) (width 0.25) (layer "B.Cu") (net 5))
 (segment (start 125.572882 119.5451) (end 127.0254 119.5451) (width 0.25) (layer "B.Cu") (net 5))
 (segment (start 125.56 119.532218) (end 125.572882 119.5451) (width 0.25) (layer "B.Cu") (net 5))
 (segment (start 120.35 119.5) (end 120 119.85) (width 0.25) (layer "B.Cu") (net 5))
 (segment (start 121.1396 119.5) (end 120.35 119.5) (width 0.25) (layer "B.Cu") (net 5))
 (segment (start 116.6 119.55) (end 115.2222 119.55) (width 0.25) (layer "B.Cu") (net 5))
 (segment (start 121.4 119.55) (end 121.35 119.5) (width 0.25) (layer "B.Cu") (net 5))
 (segment (start 122.75 119.55) (end 121.4 119.55) (width 0.25) (layer "B.Cu") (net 5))
 (segment (start 120 119.85) (end 116.9 119.85) (width 0.25) (layer "B.Cu") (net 5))
 (segment (start 123.7 110.6) (end 119.5 110.6) (width 0.25) (layer "F.Cu") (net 1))
 (segment (start 118.55 111.55) (end 118.55 118.3087) (width 0.25) (layer "F.Cu") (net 1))
 (segment (start 119.5 110.6) (end 118.55 111.55) (width 0.25) (layer "F.Cu") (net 1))
 (segment (start 125.2 109.1) (end 123.7 110.6) (width 0.25) (layer "F.Cu") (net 1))
 (segment (start 118.5799 118.3386) (end 118.5799 118.3894) (width 0.25) (layer "F.Cu") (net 1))
 (segment (start 118.55 118.3087) (end 118.5799 118.3386) (width 0.25) (layer "F.Cu") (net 1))
 (via (at 125.2 109.1) (size 0.8) (drill 0.4) (layers "F.Cu" "B.Cu") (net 1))
 (segment (start 125.25216 109.1) (end 126.9 107.45216) (width 0.25) (layer "B.Cu") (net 1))
 (segment (start 118.5913 118.35) (end 122.6 118.35) (width 0.25) (layer "B.Cu") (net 1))
 (segment (start 123.4268 119.1768) (end 124.4092 119.1768) (width 0.25) (layer "B.Cu") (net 1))
 (segment (start 122.6 118.35) (end 123.4268 119.1768) (width 0.25) (layer "B.Cu") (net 1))
 (segment (start 118.5799 118.3386) (end 118.5913 118.35) (width 0.25) (layer "B.Cu") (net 1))
 (segment (start 118.4529 118.2624) (end 118.5291 118.3386) (width 0.25) (layer "B.Cu") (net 1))
 (segment (start 118.5291 118.3386) (end 118.5799 118.3386) (width 0.25) (layer "B.Cu") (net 1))
 (segment (start 125.2 109.1) (end 125.25216 109.1) (width 0.25) (layer "B.Cu") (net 1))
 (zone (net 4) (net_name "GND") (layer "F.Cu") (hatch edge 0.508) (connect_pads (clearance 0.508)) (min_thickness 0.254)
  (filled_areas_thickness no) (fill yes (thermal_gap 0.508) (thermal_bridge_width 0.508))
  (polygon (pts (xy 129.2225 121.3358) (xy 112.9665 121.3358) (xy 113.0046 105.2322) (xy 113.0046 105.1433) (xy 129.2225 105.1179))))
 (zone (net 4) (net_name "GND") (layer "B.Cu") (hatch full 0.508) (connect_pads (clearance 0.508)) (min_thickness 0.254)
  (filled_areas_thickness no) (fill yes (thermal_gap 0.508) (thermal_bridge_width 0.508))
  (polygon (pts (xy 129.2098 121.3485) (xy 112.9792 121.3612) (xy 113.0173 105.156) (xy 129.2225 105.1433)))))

